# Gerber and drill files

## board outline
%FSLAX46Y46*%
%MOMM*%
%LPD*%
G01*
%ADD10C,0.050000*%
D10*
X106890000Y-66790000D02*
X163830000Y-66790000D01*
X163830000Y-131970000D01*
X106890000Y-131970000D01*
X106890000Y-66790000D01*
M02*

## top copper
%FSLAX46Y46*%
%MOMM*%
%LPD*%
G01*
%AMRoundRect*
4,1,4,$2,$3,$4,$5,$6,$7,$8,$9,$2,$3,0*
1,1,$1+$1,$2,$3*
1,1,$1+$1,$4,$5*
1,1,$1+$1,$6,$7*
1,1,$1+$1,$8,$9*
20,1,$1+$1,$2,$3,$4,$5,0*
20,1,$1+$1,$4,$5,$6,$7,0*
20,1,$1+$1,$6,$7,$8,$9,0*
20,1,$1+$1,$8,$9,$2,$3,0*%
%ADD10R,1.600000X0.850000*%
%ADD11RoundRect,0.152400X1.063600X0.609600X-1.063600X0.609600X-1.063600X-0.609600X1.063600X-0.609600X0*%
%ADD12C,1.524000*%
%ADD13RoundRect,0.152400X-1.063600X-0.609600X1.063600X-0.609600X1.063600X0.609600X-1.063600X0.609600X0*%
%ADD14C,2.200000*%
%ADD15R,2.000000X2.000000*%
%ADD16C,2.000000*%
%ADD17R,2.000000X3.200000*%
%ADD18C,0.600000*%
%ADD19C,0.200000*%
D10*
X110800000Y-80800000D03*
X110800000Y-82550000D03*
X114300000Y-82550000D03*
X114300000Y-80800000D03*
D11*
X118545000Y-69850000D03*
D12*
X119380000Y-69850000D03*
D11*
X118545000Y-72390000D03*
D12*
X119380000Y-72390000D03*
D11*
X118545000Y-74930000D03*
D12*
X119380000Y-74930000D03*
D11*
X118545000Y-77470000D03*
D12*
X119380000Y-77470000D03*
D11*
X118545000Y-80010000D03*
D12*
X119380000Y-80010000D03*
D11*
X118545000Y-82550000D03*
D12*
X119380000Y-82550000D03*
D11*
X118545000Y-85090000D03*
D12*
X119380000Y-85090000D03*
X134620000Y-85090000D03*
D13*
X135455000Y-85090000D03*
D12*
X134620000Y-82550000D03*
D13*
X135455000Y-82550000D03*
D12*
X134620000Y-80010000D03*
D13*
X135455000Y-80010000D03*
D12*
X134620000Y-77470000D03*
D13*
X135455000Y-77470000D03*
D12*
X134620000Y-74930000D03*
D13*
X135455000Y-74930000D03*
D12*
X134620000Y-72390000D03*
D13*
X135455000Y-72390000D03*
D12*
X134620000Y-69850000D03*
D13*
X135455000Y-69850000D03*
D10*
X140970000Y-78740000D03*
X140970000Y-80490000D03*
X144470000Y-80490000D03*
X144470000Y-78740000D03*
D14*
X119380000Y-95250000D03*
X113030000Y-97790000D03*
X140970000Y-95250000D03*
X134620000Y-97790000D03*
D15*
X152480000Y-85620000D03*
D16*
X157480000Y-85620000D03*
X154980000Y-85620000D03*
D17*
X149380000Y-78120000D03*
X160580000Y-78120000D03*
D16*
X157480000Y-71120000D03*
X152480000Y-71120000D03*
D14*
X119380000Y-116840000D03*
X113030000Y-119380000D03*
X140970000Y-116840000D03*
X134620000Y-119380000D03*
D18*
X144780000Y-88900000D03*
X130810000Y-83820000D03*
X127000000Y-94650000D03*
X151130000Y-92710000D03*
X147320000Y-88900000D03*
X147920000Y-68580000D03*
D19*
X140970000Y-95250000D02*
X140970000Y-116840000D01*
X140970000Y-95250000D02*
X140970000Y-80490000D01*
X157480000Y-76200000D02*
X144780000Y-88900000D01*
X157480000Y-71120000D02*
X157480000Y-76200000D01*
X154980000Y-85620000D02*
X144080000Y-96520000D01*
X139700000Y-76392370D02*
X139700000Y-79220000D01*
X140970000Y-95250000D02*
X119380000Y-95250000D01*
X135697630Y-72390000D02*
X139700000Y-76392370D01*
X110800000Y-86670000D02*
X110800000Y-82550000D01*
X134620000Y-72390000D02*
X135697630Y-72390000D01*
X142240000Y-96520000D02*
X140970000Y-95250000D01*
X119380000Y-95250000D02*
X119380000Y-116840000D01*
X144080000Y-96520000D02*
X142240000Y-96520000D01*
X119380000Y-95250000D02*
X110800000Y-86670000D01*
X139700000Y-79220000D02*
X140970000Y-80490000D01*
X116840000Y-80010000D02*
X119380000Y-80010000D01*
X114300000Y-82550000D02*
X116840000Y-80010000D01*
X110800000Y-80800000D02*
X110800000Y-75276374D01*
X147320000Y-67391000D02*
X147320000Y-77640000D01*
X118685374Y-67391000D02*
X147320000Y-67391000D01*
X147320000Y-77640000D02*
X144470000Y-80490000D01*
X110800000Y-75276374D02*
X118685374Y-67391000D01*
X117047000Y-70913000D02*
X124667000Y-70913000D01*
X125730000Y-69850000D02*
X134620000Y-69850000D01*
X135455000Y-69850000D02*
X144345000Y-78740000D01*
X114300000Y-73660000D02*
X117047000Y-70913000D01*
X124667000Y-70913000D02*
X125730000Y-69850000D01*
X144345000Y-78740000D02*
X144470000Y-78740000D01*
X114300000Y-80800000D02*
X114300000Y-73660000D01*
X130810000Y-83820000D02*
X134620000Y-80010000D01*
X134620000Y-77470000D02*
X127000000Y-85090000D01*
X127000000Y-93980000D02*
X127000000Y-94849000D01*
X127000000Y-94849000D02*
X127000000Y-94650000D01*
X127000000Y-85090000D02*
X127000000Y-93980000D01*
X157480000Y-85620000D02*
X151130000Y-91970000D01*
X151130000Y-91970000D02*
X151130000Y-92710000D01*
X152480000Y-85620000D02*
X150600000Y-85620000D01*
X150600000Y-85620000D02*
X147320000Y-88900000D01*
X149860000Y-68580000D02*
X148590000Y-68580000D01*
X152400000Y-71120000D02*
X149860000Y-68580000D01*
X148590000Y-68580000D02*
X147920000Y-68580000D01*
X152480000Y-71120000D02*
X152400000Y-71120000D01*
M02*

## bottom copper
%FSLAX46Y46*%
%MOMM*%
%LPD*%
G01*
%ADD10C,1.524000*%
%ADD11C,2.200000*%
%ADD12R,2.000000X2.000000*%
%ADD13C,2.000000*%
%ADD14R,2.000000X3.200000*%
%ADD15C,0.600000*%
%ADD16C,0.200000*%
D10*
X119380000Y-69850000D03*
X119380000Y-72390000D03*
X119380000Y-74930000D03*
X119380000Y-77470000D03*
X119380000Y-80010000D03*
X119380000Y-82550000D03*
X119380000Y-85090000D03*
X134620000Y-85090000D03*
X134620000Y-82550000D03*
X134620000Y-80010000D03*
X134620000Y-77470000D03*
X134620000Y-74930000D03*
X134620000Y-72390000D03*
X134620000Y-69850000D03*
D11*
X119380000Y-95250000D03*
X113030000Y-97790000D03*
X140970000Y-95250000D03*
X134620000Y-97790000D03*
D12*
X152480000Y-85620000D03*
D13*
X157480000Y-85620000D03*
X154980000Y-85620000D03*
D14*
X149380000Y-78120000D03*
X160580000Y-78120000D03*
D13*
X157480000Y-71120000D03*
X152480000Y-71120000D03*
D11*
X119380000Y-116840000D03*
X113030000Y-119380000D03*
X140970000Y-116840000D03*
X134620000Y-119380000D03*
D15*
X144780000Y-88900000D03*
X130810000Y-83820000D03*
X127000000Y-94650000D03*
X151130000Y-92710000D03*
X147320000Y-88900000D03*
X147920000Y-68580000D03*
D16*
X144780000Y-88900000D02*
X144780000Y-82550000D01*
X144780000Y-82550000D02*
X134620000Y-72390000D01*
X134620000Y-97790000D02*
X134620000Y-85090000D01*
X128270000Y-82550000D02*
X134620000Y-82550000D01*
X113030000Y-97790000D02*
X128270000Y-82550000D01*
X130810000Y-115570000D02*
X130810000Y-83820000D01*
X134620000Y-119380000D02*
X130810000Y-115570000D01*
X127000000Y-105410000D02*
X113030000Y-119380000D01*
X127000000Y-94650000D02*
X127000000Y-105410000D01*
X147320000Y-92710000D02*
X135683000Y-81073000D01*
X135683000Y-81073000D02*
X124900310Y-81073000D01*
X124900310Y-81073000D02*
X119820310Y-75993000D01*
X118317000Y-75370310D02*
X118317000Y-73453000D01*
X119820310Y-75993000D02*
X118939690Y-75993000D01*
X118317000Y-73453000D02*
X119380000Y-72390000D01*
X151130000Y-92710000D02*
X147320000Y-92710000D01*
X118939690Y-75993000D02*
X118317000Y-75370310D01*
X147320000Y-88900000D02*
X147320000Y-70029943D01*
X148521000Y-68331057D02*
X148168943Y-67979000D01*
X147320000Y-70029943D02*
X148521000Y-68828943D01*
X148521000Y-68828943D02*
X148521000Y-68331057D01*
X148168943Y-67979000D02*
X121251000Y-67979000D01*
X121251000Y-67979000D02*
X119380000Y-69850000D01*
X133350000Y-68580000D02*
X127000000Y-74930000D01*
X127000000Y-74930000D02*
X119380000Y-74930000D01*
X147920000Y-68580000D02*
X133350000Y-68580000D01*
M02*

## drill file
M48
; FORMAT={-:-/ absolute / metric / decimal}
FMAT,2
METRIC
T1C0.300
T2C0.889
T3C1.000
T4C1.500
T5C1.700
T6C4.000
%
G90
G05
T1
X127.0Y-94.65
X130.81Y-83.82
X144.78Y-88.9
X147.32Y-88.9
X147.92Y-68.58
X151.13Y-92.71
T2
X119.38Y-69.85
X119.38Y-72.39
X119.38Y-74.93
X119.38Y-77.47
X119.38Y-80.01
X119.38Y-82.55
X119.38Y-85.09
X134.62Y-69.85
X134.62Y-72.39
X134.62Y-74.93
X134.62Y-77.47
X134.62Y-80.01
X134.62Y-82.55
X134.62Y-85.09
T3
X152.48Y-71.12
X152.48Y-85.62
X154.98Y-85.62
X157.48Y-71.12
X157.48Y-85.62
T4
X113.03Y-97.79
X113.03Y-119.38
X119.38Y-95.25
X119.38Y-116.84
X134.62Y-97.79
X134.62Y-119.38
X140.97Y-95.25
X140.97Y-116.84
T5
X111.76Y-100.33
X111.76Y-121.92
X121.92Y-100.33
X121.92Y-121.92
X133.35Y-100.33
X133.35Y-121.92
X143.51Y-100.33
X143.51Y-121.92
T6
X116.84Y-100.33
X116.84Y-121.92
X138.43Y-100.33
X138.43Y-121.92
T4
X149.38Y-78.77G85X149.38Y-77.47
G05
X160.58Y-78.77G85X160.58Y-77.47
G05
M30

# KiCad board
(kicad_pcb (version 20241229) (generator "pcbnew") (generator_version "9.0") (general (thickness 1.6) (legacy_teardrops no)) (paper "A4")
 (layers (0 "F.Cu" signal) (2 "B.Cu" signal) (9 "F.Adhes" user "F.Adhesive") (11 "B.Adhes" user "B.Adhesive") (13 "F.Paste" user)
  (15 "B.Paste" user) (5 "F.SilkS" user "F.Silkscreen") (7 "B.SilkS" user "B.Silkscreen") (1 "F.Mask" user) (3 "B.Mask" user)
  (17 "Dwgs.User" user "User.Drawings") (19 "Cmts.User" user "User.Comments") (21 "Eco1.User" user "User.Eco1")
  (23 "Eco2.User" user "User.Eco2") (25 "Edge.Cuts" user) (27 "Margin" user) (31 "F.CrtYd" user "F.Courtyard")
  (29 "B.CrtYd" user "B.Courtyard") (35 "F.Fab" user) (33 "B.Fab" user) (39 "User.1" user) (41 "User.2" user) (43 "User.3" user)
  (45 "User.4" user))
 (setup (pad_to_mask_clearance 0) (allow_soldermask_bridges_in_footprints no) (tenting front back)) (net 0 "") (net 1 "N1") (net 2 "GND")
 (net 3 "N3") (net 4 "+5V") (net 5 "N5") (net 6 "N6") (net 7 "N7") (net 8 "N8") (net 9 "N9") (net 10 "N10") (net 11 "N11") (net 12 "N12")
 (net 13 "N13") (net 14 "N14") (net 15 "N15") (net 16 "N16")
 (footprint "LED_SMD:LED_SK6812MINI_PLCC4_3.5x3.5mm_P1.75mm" (layer "F.Cu") (at 112.55 81.675)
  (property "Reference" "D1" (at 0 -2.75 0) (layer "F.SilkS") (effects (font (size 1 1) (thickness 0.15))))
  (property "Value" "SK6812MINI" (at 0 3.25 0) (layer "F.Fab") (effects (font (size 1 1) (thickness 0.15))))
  (pad "1" smd rect (at -1.75 -0.875) (size 1.6 0.85) (layers "F.Cu" "F.Mask" "F.Paste") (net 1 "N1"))
  (pad "2" smd rect (at -1.75 0.875) (size 1.6 0.85) (layers "F.Cu" "F.Mask" "F.Paste") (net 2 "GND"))
  (pad "3" smd rect (at 1.75 0.875) (size 1.6 0.85) (layers "F.Cu" "F.Mask" "F.Paste") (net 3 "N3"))
  (pad "4" smd rect (at 1.75 -0.875) (size 1.6 0.85) (layers "F.Cu" "F.Mask" "F.Paste") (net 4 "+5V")))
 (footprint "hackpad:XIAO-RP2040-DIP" (layer "F.Cu") (at 127 77.47)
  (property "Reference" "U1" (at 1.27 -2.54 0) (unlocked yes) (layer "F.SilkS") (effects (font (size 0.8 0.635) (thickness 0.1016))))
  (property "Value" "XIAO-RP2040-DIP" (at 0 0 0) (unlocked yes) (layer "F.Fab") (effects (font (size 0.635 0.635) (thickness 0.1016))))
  (pad "1" smd roundrect (at -8.455 -7.62 180) (size 2.432 1.524) (layers "F.Cu" "F.Mask") (roundrect_rratio 0.1) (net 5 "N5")
   (thermal_bridge_angle 45))
  (pad "1" thru_hole circle (at -7.62 -7.62 180) (size 1.524 1.524) (drill 0.889) (layers "*.Cu" "*.Mask") (remove_unused_layers no)
   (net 5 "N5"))
  (pad "2" smd roundrect (at -8.455 -5.08 180) (size 2.432 1.524) (layers "F.Cu" "F.Mask") (roundrect_rratio 0.1) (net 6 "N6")
   (thermal_bridge_angle 45))
  (pad "2" thru_hole circle (at -7.62 -5.08 180) (size 1.524 1.524) (drill 0.889) (layers "*.Cu" "*.Mask") (remove_unused_layers no)
   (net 6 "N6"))
  (pad "3" smd roundrect (at -8.455 -2.54 180) (size 2.432 1.524) (layers "F.Cu" "F.Mask") (roundrect_rratio 0.1) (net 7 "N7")
   (thermal_bridge_angle 45))
  (pad "3" thru_hole circle (at -7.62 -2.54 180) (size 1.524 1.524) (drill 0.889) (layers "*.Cu" "*.Mask") (remove_unused_layers no)
   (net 7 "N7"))
  (pad "4" smd roundrect (at -8.455 0 180) (size 2.432 1.524) (layers "F.Cu" "F.Mask") (roundrect_rratio 0.1) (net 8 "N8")
   (thermal_bridge_angle 45))
  (pad "4" thru_hole circle (at -7.62 0 180) (size 1.524 1.524) (drill 0.889) (layers "*.Cu" "*.Mask") (remove_unused_layers no)
   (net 8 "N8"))
  (pad "5" smd roundrect (at -8.455 2.54 180) (size 2.432 1.524) (layers "F.Cu" "F.Mask") (roundrect_rratio 0.1) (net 3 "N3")
   (thermal_bridge_angle 45))
  (pad "5" thru_hole circle (at -7.62 2.54 180) (size 1.524 1.524) (drill 0.889) (layers "*.Cu" "*.Mask") (remove_unused_layers no)
   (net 3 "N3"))
  (pad "6" smd roundrect (at -8.455 5.08 180) (size 2.432 1.524) (layers "F.Cu" "F.Mask") (roundrect_rratio 0.1) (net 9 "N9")
   (thermal_bridge_angle 45))
  (pad "6" thru_hole circle (at -7.62 5.08 180) (size 1.524 1.524) (drill 0.889) (layers "*.Cu" "*.Mask") (remove_unused_layers no)
   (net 9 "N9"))
  (pad "7" smd roundrect (at -8.455 7.62 180) (size 2.432 1.524) (layers "F.Cu" "F.Mask") (roundrect_rratio 0.1) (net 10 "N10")
   (thermal_bridge_angle 45))
  (pad "7" thru_hole circle (at -7.62 7.62 180) (size 1.524 1.524) (drill 0.889) (layers "*.Cu" "*.Mask") (remove_unused_layers no)
   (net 10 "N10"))
  (pad "8" thru_hole circle (at 7.62 7.62) (size 1.524 1.524) (drill 0.889) (layers "*.Cu" "*.Mask") (remove_unused_layers no)
   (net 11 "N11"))
  (pad "8" smd roundrect (at 8.455 7.62) (size 2.432 1.524) (layers "F.Cu" "F.Mask") (roundrect_rratio 0.1) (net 11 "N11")
   (thermal_bridge_angle 45))
  (pad "9" thru_hole circle (at 7.62 5.08) (size 1.524 1.524) (drill 0.889) (layers "*.Cu" "*.Mask") (remove_unused_layers no)
   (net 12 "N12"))
  (pad "9" smd roundrect (at 8.455 5.08) (size 2.432 1.524) (layers "F.Cu" "F.Mask") (roundrect_rratio 0.1) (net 12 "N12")
   (thermal_bridge_angle 45))
  (pad "10" thru_hole circle (at 7.62 2.54) (size 1.524 1.524) (drill 0.889) (layers "*.Cu" "*.Mask") (remove_unused_layers no)
   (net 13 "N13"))
  (pad "10" smd roundrect (at 8.455 2.54) (size 2.432 1.524) (layers "F.Cu" "F.Mask") (roundrect_rratio 0.1) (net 13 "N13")
   (thermal_bridge_angle 45))
  (pad "11" thru_hole circle (at 7.62 0) (size 1.524 1.524) (drill 0.889) (layers "*.Cu" "*.Mask") (remove_unused_layers no) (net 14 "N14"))
  (pad "11" smd roundrect (at 8.455 0) (size 2.432 1.524) (layers "F.Cu" "F.Mask") (roundrect_rratio 0.1) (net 14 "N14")
   (thermal_bridge_angle 45))
  (pad "12" thru_hole circle (at 7.62 -2.54) (size 1.524 1.524) (drill 0.889) (layers "*.Cu" "*.Mask") (remove_unused_layers no)
   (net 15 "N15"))
  (pad "12" smd roundrect (at 8.455 -2.54) (size 2.432 1.524) (layers "F.Cu" "F.Mask") (roundrect_rratio 0.1) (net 15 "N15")
   (thermal_bridge_angle 45))
  (pad "13" thru_hole circle (at 7.62 -5.08) (size 1.524 1.524) (drill 0.889) (layers "*.Cu" "*.Mask") (remove_unused_layers no)
   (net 2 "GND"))
  (pad "13" smd roundrect (at 8.455 -5.08) (size 2.432 1.524) (layers "F.Cu" "F.Mask") (roundrect_rratio 0.1) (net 2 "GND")
   (thermal_bridge_angle 45))
  (pad "14" thru_hole circle (at 7.62 -7.62) (size 1.524 1.524) (drill 0.889) (layers "*.Cu" "*.Mask") (remove_unused_layers no)
   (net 4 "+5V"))
  (pad "14" smd roundrect (at 8.455 -7.62) (size 2.432 1.524) (layers "F.Cu" "F.Mask") (roundrect_rratio 0.1) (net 4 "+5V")
   (thermal_bridge_angle 45)))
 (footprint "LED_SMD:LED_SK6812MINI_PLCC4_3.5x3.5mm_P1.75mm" (layer "F.Cu") (at 142.72 79.615)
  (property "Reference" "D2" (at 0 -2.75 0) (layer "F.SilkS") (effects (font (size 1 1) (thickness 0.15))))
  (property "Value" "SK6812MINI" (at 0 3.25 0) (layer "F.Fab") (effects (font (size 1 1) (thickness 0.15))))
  (pad "1" smd rect (at -1.75 -0.875) (size 1.6 0.85) (layers "F.Cu" "F.Mask" "F.Paste") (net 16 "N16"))
  (pad "2" smd rect (at -1.75 0.875) (size 1.6 0.85) (layers "F.Cu" "F.Mask" "F.Paste") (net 2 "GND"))
  (pad "3" smd rect (at 1.75 0.875) (size 1.6 0.85) (layers "F.Cu" "F.Mask" "F.Paste") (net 1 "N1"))
  (pad "4" smd rect (at 1.75 -0.875) (size 1.6 0.85) (layers "F.Cu" "F.Mask" "F.Paste") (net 4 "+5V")))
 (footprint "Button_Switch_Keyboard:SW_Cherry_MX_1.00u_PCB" (layer "F.Cu") (at 119.38 95.25)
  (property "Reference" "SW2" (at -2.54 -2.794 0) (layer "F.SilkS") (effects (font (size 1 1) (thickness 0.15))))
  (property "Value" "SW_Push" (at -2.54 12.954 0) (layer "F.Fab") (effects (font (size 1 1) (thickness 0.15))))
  (pad "" np_thru_hole circle (at -7.62 5.08) (size 1.7 1.7) (drill 1.7) (layers "*.Cu" "*.Mask"))
  (pad "" np_thru_hole circle (at -2.54 5.08) (size 4 4) (drill 4) (layers "*.Cu" "*.Mask"))
  (pad "" np_thru_hole circle (at 2.54 5.08) (size 1.7 1.7) (drill 1.7) (layers "*.Cu" "*.Mask"))
  (pad "1" thru_hole circle (at 0 0) (size 2.2 2.2) (drill 1.5) (layers "*.Cu" "*.Mask") (remove_unused_layers no) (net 2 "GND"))
  (pad "2" thru_hole circle (at -6.35 2.54) (size 2.2 2.2) (drill 1.5) (layers "*.Cu" "*.Mask") (remove_unused_layers no) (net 12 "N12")))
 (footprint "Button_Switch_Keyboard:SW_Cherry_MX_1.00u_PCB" (layer "F.Cu") (at 140.97 95.25)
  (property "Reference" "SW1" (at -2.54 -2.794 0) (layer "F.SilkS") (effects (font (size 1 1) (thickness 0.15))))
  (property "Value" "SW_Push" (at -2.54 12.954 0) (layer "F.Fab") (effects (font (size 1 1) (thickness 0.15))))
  (pad "" np_thru_hole circle (at -7.62 5.08) (size 1.7 1.7) (drill 1.7) (layers "*.Cu" "*.Mask"))
  (pad "" np_thru_hole circle (at -2.54 5.08) (size 4 4) (drill 4) (layers "*.Cu" "*.Mask"))
  (pad "" np_thru_hole circle (at 2.54 5.08) (size 1.7 1.7) (drill 1.7) (layers "*.Cu" "*.Mask"))
  (pad "1" thru_hole circle (at 0 0) (size 2.2 2.2) (drill 1.5) (layers "*.Cu" "*.Mask") (remove_unused_layers no) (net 2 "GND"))
  (pad "2" thru_hole circle (at -6.35 2.54) (size 2.2 2.2) (drill 1.5) (layers "*.Cu" "*.Mask") (remove_unused_layers no) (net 11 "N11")))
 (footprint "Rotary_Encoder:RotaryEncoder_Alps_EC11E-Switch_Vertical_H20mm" (layer "F.Cu") (at 152.48 85.62 90)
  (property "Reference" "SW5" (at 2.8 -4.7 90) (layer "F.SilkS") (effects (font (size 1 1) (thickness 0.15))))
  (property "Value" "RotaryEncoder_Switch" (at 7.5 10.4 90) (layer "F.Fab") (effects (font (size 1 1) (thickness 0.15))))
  (pad "A" thru_hole rect (at 0 0 90) (size 2 2) (drill 1) (layers "*.Cu" "*.Mask") (remove_unused_layers no) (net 5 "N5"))
  (pad "B" thru_hole circle (at 0 5 90) (size 2 2) (drill 1) (layers "*.Cu" "*.Mask") (remove_unused_layers no) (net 6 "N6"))
  (pad "C" thru_hole circle (at 0 2.5 90) (size 2 2) (drill 1) (layers "*.Cu" "*.Mask") (remove_unused_layers no) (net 2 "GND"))
  (pad "MP" thru_hole rect (at 7.5 -3.1 90) (size 3.2 2) (drill oval 2.8 1.5) (layers "*.Cu" "*.Mask") (remove_unused_layers no))
  (pad "MP" thru_hole rect (at 7.5 8.1 90) (size 3.2 2) (drill oval 2.8 1.5) (layers "*.Cu" "*.Mask") (remove_unused_layers no))
  (pad "S1" thru_hole circle (at 14.5 5 90) (size 2 2) (drill 1) (layers "*.Cu" "*.Mask") (remove_unused_layers no) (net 2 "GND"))
  (pad "S2" thru_hole circle (at 14.5 0 90) (size 2 2) (drill 1) (layers "*.Cu" "*.Mask") (remove_unused_layers no) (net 7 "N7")))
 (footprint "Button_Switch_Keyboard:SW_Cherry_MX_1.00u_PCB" (layer "F.Cu") (at 119.38 116.84)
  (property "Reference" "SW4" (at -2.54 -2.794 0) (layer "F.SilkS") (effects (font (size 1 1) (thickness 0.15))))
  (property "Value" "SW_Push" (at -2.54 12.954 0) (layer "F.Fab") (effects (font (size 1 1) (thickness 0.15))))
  (pad "" np_thru_hole circle (at -7.62 5.08) (size 1.7 1.7) (drill 1.7) (layers "*.Cu" "*.Mask"))
  (pad "" np_thru_hole circle (at -2.54 5.08) (size 4 4) (drill 4) (layers "*.Cu" "*.Mask"))
  (pad "" np_thru_hole circle (at 2.54 5.08) (size 1.7 1.7) (drill 1.7) (layers "*.Cu" "*.Mask"))
  (pad "1" thru_hole circle (at 0 0) (size 2.2 2.2) (drill 1.5) (layers "*.Cu" "*.Mask") (remove_unused_layers no) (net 2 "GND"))
  (pad "2" thru_hole circle (at -6.35 2.54) (size 2.2 2.2) (drill 1.5) (layers "*.Cu" "*.Mask") (remove_unused_layers no) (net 14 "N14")))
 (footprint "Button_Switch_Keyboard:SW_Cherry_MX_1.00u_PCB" (layer "F.Cu") (at 140.97 116.84)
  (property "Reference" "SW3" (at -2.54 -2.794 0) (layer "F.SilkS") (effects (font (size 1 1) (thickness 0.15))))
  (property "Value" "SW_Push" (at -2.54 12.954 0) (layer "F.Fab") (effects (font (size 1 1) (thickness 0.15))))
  (pad "" np_thru_hole circle (at -7.62 5.08) (size 1.7 1.7) (drill 1.7) (layers "*.Cu" "*.Mask"))
  (pad "" np_thru_hole circle (at -2.54 5.08) (size 4 4) (drill 4) (layers "*.Cu" "*.Mask"))
  (pad "" np_thru_hole circle (at 2.54 5.08) (size 1.7 1.7) (drill 1.7) (layers "*.Cu" "*.Mask"))
  (pad "1" thru_hole circle (at 0 0) (size 2.2 2.2) (drill 1.5) (layers "*.Cu" "*.Mask") (remove_unused_layers no) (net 2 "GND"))
  (pad "2" thru_hole circle (at -6.35 2.54) (size 2.2 2.2) (drill 1.5) (layers "*.Cu" "*.Mask") (remove_unused_layers no) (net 13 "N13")))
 (gr_rect (start 106.89 66.79) (end 163.83 131.97) (stroke (width 0.05) (type solid)) (fill no) (layer "Edge.Cuts"))
 (segment (start 140.97 95.25) (end 140.97 116.84) (width 0.2) (layer "F.Cu") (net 2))
 (segment (start 140.97 95.25) (end 140.97 80.49) (width 0.2) (layer "F.Cu") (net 2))
 (segment (start 157.48 76.2) (end 144.78 88.9) (width 0.2) (layer "F.Cu") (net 2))
 (segment (start 157.48 71.12) (end 157.48 76.2) (width 0.2) (layer "F.Cu") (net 2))
 (segment (start 154.98 85.62) (end 144.08 96.52) (width 0.2) (layer "F.Cu") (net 2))
 (segment (start 139.7 76.39237) (end 139.7 79.22) (width 0.2) (layer "F.Cu") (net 2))
 (segment (start 140.97 95.25) (end 119.38 95.25) (width 0.2) (layer "F.Cu") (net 2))
 (segment (start 135.69763 72.39) (end 139.7 76.39237) (width 0.2) (layer "F.Cu") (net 2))
 (segment (start 110.8 86.67) (end 110.8 82.55) (width 0.2) (layer "F.Cu") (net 2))
 (segment (start 134.62 72.39) (end 135.69763 72.39) (width 0.2) (layer "F.Cu") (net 2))
 (segment (start 142.24 96.52) (end 140.97 95.25) (width 0.2) (layer "F.Cu") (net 2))
 (segment (start 119.38 95.25) (end 119.38 116.84) (width 0.2) (layer "F.Cu") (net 2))
 (segment (start 144.08 96.52) (end 142.24 96.52) (width 0.2) (layer "F.Cu") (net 2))
 (segment (start 119.38 95.25) (end 110.8 86.67) (width 0.2) (layer "F.Cu") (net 2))
 (segment (start 139.7 79.22) (end 140.97 80.49) (width 0.2) (layer "F.Cu") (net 2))
 (via (at 144.78 88.9) (size 0.6) (drill 0.3) (layers "F.Cu" "B.Cu") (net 2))
 (segment (start 144.78 88.9) (end 144.78 82.55) (width 0.2) (layer "B.Cu") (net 2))
 (segment (start 144.78 82.55) (end 134.62 72.39) (width 0.2) (layer "B.Cu") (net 2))
 (segment (start 116.84 80.01) (end 119.38 80.01) (width 0.2) (layer "F.Cu") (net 3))
 (segment (start 114.3 82.55) (end 116.84 80.01) (width 0.2) (layer "F.Cu") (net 3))
 (segment (start 110.8 80.8) (end 110.8 75.276374) (width 0.2) (layer "F.Cu") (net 1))
 (segment (start 147.32 67.391) (end 147.32 77.64) (width 0.2) (layer "F.Cu") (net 1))
 (segment (start 118.685374 67.391) (end 147.32 67.391) (width 0.2) (layer "F.Cu") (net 1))
 (segment (start 147.32 77.64) (end 144.47 80.49) (width 0.2) (layer "F.Cu") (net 1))
 (segment (start 110.8 75.276374) (end 118.685374 67.391) (width 0.2) (layer "F.Cu") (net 1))
 (segment (start 117.047 70.913) (end 124.667 70.913) (width 0.2) (layer "F.Cu") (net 4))
 (segment (start 125.73 69.85) (end 134.62 69.85) (width 0.2) (layer "F.Cu") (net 4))
 (segment (start 135.455 69.85) (end 144.345 78.74) (width 0.2) (layer "F.Cu") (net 4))
 (segment (start 114.3 73.66) (end 117.047 70.913) (width 0.2) (layer "F.Cu") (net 4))
 (segment (start 124.667 70.913) (end 125.73 69.85) (width 0.2) (layer "F.Cu") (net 4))
 (segment (start 144.345 78.74) (end 144.47 78.74) (width 0.2) (layer "F.Cu") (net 4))
 (segment (start 114.3 80.8) (end 114.3 73.66) (width 0.2) (layer "F.Cu") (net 4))
 (segment (start 134.62 97.79) (end 134.62 85.09) (width 0.2) (layer "B.Cu") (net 11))
 (segment (start 128.27 82.55) (end 134.62 82.55) (width 0.2) (layer "B.Cu") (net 12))
 (segment (start 113.03 97.79) (end 128.27 82.55) (width 0.2) (layer "B.Cu") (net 12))
 (segment (start 130.81 83.82) (end 134.62 80.01) (width 0.2) (layer "F.Cu") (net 13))
 (via (at 130.81 83.82) (size 0.6) (drill 0.3) (layers "F.Cu" "B.Cu") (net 13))
 (segment (start 130.81 115.57) (end 130.81 83.82) (width 0.2) (layer "B.Cu") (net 13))
 (segment (start 134.62 119.38) (end 130.81 115.57) (width 0.2) (layer "B.Cu") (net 13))
 (segment (start 134.62 77.47) (end 127 85.09) (width 0.2) (layer "F.Cu") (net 14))
 (segment (start 127 93.98) (end 127 94.849) (width 0.2) (layer "F.Cu") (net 14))
 (segment (start 127 94.849) (end 127 94.65) (width 0.2) (layer "F.Cu") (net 14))
 (segment (start 127 85.09) (end 127 93.98) (width 0.2) (layer "F.Cu") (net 14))
 (via (at 127 94.65) (size 0.6) (drill 0.3) (layers "F.Cu" "B.Cu") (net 14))
 (segment (start 127 105.41) (end 113.03 119.38) (width 0.2) (layer "B.Cu") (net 14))
 (segment (start 127 94.65) (end 127 105.41) (width 0.2) (layer "B.Cu") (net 14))
 (segment (start 157.48 85.62) (end 151.13 91.97) (width 0.2) (layer "F.Cu") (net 6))
 (segment (start 151.13 91.97) (end 151.13 92.71) (width 0.2) (layer "F.Cu") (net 6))
 (via (at 151.13 92.71) (size 0.6) (drill 0.3) (layers "F.Cu" "B.Cu") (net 6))
 (segment (start 147.32 92.71) (end 135.683 81.073) (width 0.2) (layer "B.Cu") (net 6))
 (segment (start 135.683 81.073) (end 124.90031 81.073) (width 0.2) (layer "B.Cu") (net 6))
 (segment (start 124.90031 81.073) (end 119.82031 75.993) (width 0.2) (layer "B.Cu") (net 6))
 (segment (start 118.317 75.37031) (end 118.317 73.453) (width 0.2) (layer "B.Cu") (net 6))
 (segment (start 119.82031 75.993) (end 118.93969 75.993) (width 0.2) (layer "B.Cu") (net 6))
 (segment (start 118.317 73.453) (end 119.38 72.39) (width 0.2) (layer "B.Cu") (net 6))
 (segment (start 151.13 92.71) (end 147.32 92.71) (width 0.2) (layer "B.Cu") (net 6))
 (segment (start 118.93969 75.993) (end 118.317 75.37031) (width 0.2) (layer "B.Cu") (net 6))
 (segment (start 152.48 85.62) (end 150.6 85.62) (width 0.2) (layer "F.Cu") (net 5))
 (segment (start 150.6 85.62) (end 147.32 88.9) (width 0.2) (layer "F.Cu") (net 5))
 (via (at 147.32 88.9) (size 0.6) (drill 0.3) (layers "F.Cu" "B.Cu") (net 5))
 (segment (start 147.32 88.9) (end 147.32 70.029943) (width 0.2) (layer "B.Cu") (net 5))
 (segment (start 148.521 68.331057) (end 148.168943 67.979) (width 0.2) (layer "B.Cu") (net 5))
 (segment (start 147.32 70.029943) (end 148.521 68.828943) (width 0.2) (layer "B.Cu") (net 5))
 (segment (start 148.521 68.828943) (end 148.521 68.331057) (width 0.2) (layer "B.Cu") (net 5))
 (segment (start 148.168943 67.979) (end 121.251 67.979) (width 0.2) (layer "B.Cu") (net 5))
 (segment (start 121.251 67.979) (end 119.38 69.85) (width 0.2) (layer "B.Cu") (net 5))
 (segment (start 149.86 68.58) (end 148.59 68.58) (width 0.2) (layer "F.Cu") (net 7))
 (segment (start 152.4 71.12) (end 149.86 68.58) (width 0.2) (layer "F.Cu") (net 7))
 (segment (start 148.59 68.58) (end 147.92 68.58) (width 0.2) (layer "F.Cu") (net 7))
 (segment (start 152.48 71.12) (end 152.4 71.12) (width 0.2) (layer "F.Cu") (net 7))
 (via (at 147.92 68.58) (size 0.6) (drill 0.3) (layers "F.Cu" "B.Cu") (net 7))
 (segment (start 133.35 68.58) (end 127 74.93) (width 0.2) (layer "B.Cu") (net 7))
 (segment (start 127 74.93) (end 119.38 74.93) (width 0.2) (layer "B.Cu") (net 7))
 (segment (start 147.92 68.58) (end 133.35 68.58) (width 0.2) (layer "B.Cu") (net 7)))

